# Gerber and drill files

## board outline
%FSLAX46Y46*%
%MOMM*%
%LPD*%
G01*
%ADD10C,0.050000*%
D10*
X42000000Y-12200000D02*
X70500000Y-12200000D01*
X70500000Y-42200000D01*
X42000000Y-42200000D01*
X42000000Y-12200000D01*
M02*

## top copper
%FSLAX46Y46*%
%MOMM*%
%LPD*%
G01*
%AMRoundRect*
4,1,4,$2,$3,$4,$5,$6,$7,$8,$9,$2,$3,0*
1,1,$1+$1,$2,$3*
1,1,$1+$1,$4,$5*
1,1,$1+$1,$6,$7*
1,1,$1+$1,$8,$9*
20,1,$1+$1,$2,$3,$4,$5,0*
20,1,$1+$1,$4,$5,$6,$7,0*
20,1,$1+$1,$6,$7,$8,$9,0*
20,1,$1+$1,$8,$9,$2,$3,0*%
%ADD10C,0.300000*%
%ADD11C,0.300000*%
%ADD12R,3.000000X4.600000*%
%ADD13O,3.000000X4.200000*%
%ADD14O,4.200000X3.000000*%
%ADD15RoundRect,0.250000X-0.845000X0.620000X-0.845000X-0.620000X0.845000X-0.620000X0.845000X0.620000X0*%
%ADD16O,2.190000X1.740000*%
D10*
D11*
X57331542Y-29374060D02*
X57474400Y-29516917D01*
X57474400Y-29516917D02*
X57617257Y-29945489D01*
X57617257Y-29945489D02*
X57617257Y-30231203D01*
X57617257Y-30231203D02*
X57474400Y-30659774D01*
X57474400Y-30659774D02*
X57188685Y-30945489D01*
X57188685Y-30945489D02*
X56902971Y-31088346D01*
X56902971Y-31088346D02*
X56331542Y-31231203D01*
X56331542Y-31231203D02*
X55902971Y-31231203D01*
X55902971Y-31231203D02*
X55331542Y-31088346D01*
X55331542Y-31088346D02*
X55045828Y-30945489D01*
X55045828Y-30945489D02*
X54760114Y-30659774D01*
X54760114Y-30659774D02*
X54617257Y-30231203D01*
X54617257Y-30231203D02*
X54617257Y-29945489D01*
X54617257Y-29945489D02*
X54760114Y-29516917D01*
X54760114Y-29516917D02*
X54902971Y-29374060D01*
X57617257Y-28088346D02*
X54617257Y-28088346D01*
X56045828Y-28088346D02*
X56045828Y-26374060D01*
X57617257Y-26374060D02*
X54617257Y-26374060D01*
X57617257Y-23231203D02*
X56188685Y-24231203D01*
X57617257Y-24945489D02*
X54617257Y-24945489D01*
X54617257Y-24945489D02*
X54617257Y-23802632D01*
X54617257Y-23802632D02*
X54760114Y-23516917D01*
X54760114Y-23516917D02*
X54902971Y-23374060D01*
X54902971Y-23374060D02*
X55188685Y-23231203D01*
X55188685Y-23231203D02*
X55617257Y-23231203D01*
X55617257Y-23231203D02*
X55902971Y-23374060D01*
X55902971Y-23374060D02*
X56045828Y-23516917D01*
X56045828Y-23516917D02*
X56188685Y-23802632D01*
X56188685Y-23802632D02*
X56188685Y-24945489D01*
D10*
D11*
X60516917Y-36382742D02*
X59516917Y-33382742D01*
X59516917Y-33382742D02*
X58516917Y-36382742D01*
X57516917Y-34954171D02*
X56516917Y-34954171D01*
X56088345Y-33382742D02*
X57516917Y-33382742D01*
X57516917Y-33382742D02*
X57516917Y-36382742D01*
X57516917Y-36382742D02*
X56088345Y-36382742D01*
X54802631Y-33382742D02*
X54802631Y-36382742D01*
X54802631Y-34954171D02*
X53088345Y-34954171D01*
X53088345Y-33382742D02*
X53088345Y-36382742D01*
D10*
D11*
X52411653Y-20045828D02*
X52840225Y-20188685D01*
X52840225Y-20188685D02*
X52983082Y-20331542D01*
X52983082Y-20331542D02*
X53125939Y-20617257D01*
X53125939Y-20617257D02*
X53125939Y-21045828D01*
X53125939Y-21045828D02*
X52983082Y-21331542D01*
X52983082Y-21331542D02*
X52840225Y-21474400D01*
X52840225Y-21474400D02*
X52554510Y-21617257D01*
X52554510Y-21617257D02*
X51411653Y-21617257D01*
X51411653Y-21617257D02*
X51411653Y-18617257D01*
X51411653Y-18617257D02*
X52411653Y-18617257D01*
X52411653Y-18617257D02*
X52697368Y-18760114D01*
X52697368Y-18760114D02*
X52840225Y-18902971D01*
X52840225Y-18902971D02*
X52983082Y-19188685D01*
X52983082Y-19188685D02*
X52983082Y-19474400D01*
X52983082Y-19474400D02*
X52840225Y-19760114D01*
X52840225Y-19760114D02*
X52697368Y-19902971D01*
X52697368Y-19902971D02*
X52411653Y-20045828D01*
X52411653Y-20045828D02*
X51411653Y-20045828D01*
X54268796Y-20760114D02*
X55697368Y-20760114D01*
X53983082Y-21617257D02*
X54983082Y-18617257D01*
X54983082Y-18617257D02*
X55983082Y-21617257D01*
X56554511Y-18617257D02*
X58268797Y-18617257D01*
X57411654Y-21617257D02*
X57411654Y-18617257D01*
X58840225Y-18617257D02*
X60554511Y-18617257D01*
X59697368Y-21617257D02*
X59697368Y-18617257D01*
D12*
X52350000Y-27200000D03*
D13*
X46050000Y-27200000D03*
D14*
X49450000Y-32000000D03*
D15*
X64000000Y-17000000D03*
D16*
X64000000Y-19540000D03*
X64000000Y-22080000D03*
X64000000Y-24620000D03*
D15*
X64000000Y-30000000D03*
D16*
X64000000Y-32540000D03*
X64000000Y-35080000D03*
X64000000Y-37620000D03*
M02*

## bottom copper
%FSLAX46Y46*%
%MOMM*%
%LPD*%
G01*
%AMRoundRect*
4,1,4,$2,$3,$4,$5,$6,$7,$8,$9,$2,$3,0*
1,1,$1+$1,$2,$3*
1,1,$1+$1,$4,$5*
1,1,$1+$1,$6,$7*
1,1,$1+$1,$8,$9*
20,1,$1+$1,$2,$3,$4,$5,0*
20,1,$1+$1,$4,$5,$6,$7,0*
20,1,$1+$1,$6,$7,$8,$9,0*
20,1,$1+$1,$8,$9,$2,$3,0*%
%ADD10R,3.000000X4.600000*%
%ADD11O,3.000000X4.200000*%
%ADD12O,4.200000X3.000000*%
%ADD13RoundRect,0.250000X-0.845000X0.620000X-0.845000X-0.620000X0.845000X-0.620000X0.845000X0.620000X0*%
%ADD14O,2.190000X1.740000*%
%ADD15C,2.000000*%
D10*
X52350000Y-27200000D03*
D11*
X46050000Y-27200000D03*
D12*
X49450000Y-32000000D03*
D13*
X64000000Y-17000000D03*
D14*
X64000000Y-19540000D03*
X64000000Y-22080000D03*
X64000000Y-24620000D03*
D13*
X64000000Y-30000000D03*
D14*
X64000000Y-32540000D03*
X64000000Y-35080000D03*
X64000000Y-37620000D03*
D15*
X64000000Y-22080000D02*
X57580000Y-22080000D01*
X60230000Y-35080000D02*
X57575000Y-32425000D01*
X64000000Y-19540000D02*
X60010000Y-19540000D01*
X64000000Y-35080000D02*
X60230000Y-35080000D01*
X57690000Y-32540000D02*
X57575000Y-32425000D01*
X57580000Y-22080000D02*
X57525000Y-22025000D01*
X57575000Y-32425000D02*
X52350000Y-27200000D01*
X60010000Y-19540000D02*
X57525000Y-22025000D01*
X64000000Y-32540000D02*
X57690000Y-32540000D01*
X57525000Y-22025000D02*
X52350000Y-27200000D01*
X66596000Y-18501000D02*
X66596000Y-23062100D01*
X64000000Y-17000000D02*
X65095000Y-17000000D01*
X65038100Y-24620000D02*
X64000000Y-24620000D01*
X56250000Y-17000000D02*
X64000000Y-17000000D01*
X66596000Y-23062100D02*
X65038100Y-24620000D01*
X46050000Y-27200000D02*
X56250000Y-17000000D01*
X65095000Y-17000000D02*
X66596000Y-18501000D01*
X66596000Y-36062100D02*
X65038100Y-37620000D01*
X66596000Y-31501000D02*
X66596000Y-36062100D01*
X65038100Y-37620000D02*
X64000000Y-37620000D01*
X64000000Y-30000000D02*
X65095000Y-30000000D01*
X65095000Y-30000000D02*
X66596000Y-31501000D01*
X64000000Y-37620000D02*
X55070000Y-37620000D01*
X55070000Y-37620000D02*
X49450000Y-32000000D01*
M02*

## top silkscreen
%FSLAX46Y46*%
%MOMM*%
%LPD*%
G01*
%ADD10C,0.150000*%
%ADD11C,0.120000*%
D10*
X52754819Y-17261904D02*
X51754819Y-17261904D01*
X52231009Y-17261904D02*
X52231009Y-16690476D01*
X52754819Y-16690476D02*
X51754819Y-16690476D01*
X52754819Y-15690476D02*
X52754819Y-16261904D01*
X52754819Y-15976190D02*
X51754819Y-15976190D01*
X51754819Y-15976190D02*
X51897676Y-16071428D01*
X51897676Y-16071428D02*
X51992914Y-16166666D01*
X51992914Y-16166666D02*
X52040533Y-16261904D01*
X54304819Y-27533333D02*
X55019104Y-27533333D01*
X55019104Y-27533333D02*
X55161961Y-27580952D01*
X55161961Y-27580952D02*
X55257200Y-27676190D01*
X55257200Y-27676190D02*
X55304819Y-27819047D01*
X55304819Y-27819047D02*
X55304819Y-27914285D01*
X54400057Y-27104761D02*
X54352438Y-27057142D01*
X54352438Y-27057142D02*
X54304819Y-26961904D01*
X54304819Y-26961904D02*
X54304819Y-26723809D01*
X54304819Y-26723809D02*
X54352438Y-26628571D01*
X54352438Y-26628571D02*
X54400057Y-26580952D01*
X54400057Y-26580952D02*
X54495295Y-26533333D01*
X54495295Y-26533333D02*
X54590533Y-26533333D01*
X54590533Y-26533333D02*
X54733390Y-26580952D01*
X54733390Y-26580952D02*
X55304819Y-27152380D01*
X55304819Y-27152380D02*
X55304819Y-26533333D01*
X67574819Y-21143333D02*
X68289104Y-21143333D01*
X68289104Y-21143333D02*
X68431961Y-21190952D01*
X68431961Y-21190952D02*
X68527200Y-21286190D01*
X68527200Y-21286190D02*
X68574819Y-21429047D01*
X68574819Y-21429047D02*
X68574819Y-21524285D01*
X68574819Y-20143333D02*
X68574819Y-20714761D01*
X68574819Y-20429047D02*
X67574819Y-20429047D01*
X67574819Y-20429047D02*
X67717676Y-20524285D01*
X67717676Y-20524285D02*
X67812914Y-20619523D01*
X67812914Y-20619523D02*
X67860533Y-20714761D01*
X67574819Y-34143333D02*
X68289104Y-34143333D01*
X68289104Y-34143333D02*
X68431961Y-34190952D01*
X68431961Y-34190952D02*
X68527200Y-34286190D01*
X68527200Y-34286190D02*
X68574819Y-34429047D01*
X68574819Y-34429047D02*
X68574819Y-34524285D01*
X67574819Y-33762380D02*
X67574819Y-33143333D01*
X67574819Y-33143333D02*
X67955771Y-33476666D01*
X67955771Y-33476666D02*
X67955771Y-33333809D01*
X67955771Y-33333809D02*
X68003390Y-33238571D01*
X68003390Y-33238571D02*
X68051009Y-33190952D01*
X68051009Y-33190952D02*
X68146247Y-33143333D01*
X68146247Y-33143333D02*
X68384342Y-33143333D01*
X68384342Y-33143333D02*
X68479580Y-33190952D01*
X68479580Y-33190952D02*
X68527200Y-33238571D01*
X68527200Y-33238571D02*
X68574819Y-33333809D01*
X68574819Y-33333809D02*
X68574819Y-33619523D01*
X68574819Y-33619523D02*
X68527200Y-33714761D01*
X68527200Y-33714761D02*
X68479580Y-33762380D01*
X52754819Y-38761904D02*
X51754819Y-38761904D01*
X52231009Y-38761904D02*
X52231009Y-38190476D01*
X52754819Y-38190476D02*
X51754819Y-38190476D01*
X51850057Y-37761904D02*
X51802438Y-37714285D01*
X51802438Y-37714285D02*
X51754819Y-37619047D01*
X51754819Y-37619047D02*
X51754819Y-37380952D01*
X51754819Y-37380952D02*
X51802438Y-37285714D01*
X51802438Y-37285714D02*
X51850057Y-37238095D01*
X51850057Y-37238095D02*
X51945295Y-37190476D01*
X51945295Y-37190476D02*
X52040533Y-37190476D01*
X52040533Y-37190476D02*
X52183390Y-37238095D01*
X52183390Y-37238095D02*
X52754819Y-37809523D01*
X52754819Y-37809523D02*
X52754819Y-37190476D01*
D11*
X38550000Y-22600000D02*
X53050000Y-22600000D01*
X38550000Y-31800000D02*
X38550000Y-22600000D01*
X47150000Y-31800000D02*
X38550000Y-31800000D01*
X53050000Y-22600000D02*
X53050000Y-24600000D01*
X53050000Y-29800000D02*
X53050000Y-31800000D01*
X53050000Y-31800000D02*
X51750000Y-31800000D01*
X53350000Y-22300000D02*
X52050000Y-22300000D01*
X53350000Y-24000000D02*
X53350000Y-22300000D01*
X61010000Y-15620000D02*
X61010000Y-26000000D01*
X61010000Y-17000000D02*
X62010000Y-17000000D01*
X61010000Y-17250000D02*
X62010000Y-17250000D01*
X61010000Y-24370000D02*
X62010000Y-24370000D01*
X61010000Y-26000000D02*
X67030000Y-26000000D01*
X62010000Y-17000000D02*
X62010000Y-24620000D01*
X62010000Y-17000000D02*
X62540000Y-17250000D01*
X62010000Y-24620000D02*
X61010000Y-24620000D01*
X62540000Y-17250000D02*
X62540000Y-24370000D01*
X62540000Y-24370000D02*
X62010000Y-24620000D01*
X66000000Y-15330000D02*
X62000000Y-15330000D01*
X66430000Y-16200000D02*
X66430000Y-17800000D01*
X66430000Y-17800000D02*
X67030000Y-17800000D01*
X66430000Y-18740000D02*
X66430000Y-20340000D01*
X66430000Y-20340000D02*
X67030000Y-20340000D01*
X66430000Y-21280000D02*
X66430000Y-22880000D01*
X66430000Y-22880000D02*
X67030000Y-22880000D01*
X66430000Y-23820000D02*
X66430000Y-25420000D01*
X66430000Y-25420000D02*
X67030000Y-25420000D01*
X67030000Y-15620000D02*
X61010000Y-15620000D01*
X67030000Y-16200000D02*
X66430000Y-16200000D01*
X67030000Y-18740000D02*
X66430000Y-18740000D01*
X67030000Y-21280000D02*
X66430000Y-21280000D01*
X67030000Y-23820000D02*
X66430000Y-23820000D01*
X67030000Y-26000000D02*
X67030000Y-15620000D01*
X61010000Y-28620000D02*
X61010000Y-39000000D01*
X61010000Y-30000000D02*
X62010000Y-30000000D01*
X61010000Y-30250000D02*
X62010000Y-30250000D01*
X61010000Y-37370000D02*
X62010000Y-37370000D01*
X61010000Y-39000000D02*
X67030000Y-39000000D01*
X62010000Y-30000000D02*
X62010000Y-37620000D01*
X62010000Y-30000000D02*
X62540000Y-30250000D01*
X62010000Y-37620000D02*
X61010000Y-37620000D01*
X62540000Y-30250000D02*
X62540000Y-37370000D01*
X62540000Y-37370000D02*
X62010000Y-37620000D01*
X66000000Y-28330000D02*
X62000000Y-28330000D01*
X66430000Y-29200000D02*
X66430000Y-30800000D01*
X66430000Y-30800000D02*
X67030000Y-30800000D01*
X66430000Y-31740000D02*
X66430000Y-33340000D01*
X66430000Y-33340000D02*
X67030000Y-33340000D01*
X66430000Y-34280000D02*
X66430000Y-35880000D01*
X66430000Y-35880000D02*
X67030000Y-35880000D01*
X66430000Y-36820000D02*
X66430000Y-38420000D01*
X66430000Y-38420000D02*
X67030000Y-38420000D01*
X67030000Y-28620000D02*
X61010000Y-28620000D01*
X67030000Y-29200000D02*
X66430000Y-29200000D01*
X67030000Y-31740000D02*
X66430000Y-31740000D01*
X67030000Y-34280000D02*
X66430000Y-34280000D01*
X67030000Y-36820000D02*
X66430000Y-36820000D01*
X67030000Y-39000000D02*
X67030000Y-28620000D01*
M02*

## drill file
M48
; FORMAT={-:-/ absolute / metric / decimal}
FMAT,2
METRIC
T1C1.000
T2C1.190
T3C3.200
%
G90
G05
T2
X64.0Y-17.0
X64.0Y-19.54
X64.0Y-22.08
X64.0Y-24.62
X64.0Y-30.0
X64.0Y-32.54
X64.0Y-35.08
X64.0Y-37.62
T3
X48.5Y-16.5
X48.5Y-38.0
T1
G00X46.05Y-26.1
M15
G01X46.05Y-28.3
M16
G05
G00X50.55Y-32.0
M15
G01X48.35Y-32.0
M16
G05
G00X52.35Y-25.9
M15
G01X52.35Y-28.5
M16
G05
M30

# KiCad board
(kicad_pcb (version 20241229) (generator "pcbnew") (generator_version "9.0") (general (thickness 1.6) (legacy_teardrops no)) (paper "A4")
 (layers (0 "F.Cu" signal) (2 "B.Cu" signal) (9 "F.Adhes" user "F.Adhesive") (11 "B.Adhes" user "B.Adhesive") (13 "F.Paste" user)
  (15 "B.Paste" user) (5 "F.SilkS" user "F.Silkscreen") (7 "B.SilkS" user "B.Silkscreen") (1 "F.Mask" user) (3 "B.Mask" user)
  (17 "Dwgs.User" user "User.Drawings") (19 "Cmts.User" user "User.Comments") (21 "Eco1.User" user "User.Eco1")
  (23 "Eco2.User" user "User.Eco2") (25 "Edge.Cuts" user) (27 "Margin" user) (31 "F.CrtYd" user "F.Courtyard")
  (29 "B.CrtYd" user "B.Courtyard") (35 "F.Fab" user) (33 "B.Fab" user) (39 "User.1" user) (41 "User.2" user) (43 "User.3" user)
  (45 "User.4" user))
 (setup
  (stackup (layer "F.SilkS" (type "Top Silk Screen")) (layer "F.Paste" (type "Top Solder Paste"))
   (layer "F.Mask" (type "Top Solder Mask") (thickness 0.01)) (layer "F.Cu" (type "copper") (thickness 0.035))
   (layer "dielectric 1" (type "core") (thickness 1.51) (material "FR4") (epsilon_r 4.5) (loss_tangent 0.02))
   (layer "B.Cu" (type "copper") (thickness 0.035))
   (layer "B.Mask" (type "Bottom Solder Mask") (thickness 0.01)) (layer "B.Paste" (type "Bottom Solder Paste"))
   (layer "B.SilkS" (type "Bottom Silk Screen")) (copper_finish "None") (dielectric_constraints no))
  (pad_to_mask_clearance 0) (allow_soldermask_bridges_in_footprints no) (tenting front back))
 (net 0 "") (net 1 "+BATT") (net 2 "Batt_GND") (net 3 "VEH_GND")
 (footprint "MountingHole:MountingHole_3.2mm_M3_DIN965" (layer "F.Cu") (at 48.5 16.5 -90)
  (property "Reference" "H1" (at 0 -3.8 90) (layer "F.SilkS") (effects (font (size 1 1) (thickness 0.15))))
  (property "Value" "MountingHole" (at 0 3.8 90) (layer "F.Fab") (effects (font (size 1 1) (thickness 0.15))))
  (pad "" np_thru_hole circle (at 0 0 270) (size 3.2 3.2) (drill 3.2) (layers "*.Cu" "*.Mask")))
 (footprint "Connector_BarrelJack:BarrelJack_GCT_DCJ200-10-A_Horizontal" (layer "F.Cu") (at 52.35 27.2 -90)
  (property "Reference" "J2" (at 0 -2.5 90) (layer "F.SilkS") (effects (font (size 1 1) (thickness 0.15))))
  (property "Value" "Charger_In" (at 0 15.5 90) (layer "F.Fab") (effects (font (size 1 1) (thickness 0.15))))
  (fp_line (start -4.6 13.8) (end -4.6 -0.7) (stroke (width 0.12) (type solid)) (layer "F.SilkS"))
  (fp_line (start 4.6 13.8) (end -4.6 13.8) (stroke (width 0.12) (type solid)) (layer "F.SilkS"))
  (fp_line (start 4.6 5.2) (end 4.6 13.8) (stroke (width 0.12) (type solid)) (layer "F.SilkS"))
  (fp_line (start -4.6 -0.7) (end -2.6 -0.7) (stroke (width 0.12) (type solid)) (layer "F.SilkS"))
  (fp_line (start 2.6 -0.7) (end 4.6 -0.7) (stroke (width 0.12) (type solid)) (layer "F.SilkS"))
  (fp_line (start 4.6 -0.7) (end 4.6 0.6) (stroke (width 0.12) (type solid)) (layer "F.SilkS"))
  (fp_line (start -4.9 -1) (end -4.9 0.3) (stroke (width 0.12) (type solid)) (layer "F.SilkS"))
  (fp_line (start -3.2 -1) (end -4.9 -1) (stroke (width 0.12) (type solid)) (layer "F.SilkS"))
  (pad "1" thru_hole rect (at 0 0 270) (size 4.6 3) (drill oval 3.6 1) (layers "*.Cu" "*.Mask") (remove_unused_layers no) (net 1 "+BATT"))
  (pad "2" thru_hole oval (at 0 6.3 270) (size 4.2 3) (drill oval 3.2 1) (layers "*.Cu" "*.Mask") (remove_unused_layers no)
   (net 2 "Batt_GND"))
  (pad "3" thru_hole oval (at 4.8 2.9 270) (size 3 4.2) (drill oval 1 3.2) (layers "*.Cu" "*.Mask") (remove_unused_layers no)
   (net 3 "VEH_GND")))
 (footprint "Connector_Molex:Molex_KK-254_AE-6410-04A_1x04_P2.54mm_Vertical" (layer "F.Cu") (at 64 17 -90)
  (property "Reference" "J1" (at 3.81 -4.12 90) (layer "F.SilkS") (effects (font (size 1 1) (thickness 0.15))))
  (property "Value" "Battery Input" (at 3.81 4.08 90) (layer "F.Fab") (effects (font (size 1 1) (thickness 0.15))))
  (fp_line (start -1.38 2.99) (end 9 2.99) (stroke (width 0.12) (type solid)) (layer "F.SilkS"))
  (fp_line (start 0 2.99) (end 0 1.99) (stroke (width 0.12) (type solid)) (layer "F.SilkS"))
  (fp_line (start 0.25 2.99) (end 0.25 1.99) (stroke (width 0.12) (type solid)) (layer "F.SilkS"))
  (fp_line (start 7.37 2.99) (end 7.37 1.99) (stroke (width 0.12) (type solid)) (layer "F.SilkS"))
  (fp_line (start 9 2.99) (end 9 -3.03) (stroke (width 0.12) (type solid)) (layer "F.SilkS"))
  (fp_line (start 0 1.99) (end 7.62 1.99) (stroke (width 0.12) (type solid)) (layer "F.SilkS"))
  (fp_line (start 0 1.99) (end 0.25 1.46) (stroke (width 0.12) (type solid)) (layer "F.SilkS"))
  (fp_line (start 7.62 1.99) (end 7.62 2.99) (stroke (width 0.12) (type solid)) (layer "F.SilkS"))
  (fp_line (start 0.25 1.46) (end 7.37 1.46) (stroke (width 0.12) (type solid)) (layer "F.SilkS"))
  (fp_line (start 7.37 1.46) (end 7.62 1.99) (stroke (width 0.12) (type solid)) (layer "F.SilkS"))
  (fp_line (start -1.67 -2) (end -1.67 2) (stroke (width 0.12) (type solid)) (layer "F.SilkS"))
  (fp_line (start -0.8 -2.43) (end 0.8 -2.43) (stroke (width 0.12) (type solid)) (layer "F.SilkS"))
  (fp_line (start 0.8 -2.43) (end 0.8 -3.03) (stroke (width 0.12) (type solid)) (layer "F.SilkS"))
  (fp_line (start 1.74 -2.43) (end 3.34 -2.43) (stroke (width 0.12) (type solid)) (layer "F.SilkS"))
  (fp_line (start 3.34 -2.43) (end 3.34 -3.03) (stroke (width 0.12) (type solid)) (layer "F.SilkS"))
  (fp_line (start 4.28 -2.43) (end 5.88 -2.43) (stroke (width 0.12) (type solid)) (layer "F.SilkS"))
  (fp_line (start 5.88 -2.43) (end 5.88 -3.03) (stroke (width 0.12) (type solid)) (layer "F.SilkS"))
  (fp_line (start 6.82 -2.43) (end 8.42 -2.43) (stroke (width 0.12) (type solid)) (layer "F.SilkS"))
  (fp_line (start 8.42 -2.43) (end 8.42 -3.03) (stroke (width 0.12) (type solid)) (layer "F.SilkS"))
  (fp_line (start -1.38 -3.03) (end -1.38 2.99) (stroke (width 0.12) (type solid)) (layer "F.SilkS"))
  (fp_line (start -0.8 -3.03) (end -0.8 -2.43) (stroke (width 0.12) (type solid)) (layer "F.SilkS"))
  (fp_line (start 1.74 -3.03) (end 1.74 -2.43) (stroke (width 0.12) (type solid)) (layer "F.SilkS"))
  (fp_line (start 4.28 -3.03) (end 4.28 -2.43) (stroke (width 0.12) (type solid)) (layer "F.SilkS"))
  (fp_line (start 6.82 -3.03) (end 6.82 -2.43) (stroke (width 0.12) (type solid)) (layer "F.SilkS"))
  (fp_line (start 9 -3.03) (end -1.38 -3.03) (stroke (width 0.12) (type solid)) (layer "F.SilkS"))
  (pad "1" thru_hole roundrect (at 0 0 270) (size 1.74 2.19) (drill 1.19) (layers "*.Cu" "*.Mask") (remove_unused_layers no)
   (roundrect_rratio 0.143678) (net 2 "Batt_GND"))
  (pad "2" thru_hole oval (at 2.54 0 270) (size 1.74 2.19) (drill 1.19) (layers "*.Cu" "*.Mask") (remove_unused_layers no) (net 1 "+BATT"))
  (pad "3" thru_hole oval (at 5.08 0 270) (size 1.74 2.19) (drill 1.19) (layers "*.Cu" "*.Mask") (remove_unused_layers no) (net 1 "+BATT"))
  (pad "4" thru_hole oval (at 7.62 0 270) (size 1.74 2.19) (drill 1.19) (layers "*.Cu" "*.Mask") (remove_unused_layers no)
   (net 2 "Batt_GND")))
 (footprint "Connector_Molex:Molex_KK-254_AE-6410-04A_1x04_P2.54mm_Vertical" (layer "F.Cu") (at 64 30 -90)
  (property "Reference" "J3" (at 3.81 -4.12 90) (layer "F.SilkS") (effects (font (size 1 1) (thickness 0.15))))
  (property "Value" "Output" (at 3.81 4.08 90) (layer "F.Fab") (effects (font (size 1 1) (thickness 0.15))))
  (fp_line (start -1.38 2.99) (end 9 2.99) (stroke (width 0.12) (type solid)) (layer "F.SilkS"))
  (fp_line (start 0 2.99) (end 0 1.99) (stroke (width 0.12) (type solid)) (layer "F.SilkS"))
  (fp_line (start 0.25 2.99) (end 0.25 1.99) (stroke (width 0.12) (type solid)) (layer "F.SilkS"))
  (fp_line (start 7.37 2.99) (end 7.37 1.99) (stroke (width 0.12) (type solid)) (layer "F.SilkS"))
  (fp_line (start 9 2.99) (end 9 -3.03) (stroke (width 0.12) (type solid)) (layer "F.SilkS"))
  (fp_line (start 0 1.99) (end 7.62 1.99) (stroke (width 0.12) (type solid)) (layer "F.SilkS"))
  (fp_line (start 0 1.99) (end 0.25 1.46) (stroke (width 0.12) (type solid)) (layer "F.SilkS"))
  (fp_line (start 7.62 1.99) (end 7.62 2.99) (stroke (width 0.12) (type solid)) (layer "F.SilkS"))
  (fp_line (start 0.25 1.46) (end 7.37 1.46) (stroke (width 0.12) (type solid)) (layer "F.SilkS"))
  (fp_line (start 7.37 1.46) (end 7.62 1.99) (stroke (width 0.12) (type solid)) (layer "F.SilkS"))
  (fp_line (start -1.67 -2) (end -1.67 2) (stroke (width 0.12) (type solid)) (layer "F.SilkS"))
  (fp_line (start -0.8 -2.43) (end 0.8 -2.43) (stroke (width 0.12) (type solid)) (layer "F.SilkS"))
  (fp_line (start 0.8 -2.43) (end 0.8 -3.03) (stroke (width 0.12) (type solid)) (layer "F.SilkS"))
  (fp_line (start 1.74 -2.43) (end 3.34 -2.43) (stroke (width 0.12) (type solid)) (layer "F.SilkS"))
  (fp_line (start 3.34 -2.43) (end 3.34 -3.03) (stroke (width 0.12) (type solid)) (layer "F.SilkS"))
  (fp_line (start 4.28 -2.43) (end 5.88 -2.43) (stroke (width 0.12) (type solid)) (layer "F.SilkS"))
  (fp_line (start 5.88 -2.43) (end 5.88 -3.03) (stroke (width 0.12) (type solid)) (layer "F.SilkS"))
  (fp_line (start 6.82 -2.43) (end 8.42 -2.43) (stroke (width 0.12) (type solid)) (layer "F.SilkS"))
  (fp_line (start 8.42 -2.43) (end 8.42 -3.03) (stroke (width 0.12) (type solid)) (layer "F.SilkS"))
  (fp_line (start -1.38 -3.03) (end -1.38 2.99) (stroke (width 0.12) (type solid)) (layer "F.SilkS"))
  (fp_line (start -0.8 -3.03) (end -0.8 -2.43) (stroke (width 0.12) (type solid)) (layer "F.SilkS"))
  (fp_line (start 1.74 -3.03) (end 1.74 -2.43) (stroke (width 0.12) (type solid)) (layer "F.SilkS"))
  (fp_line (start 4.28 -3.03) (end 4.28 -2.43) (stroke (width 0.12) (type solid)) (layer "F.SilkS"))
  (fp_line (start 6.82 -3.03) (end 6.82 -2.43) (stroke (width 0.12) (type solid)) (layer "F.SilkS"))
  (fp_line (start 9 -3.03) (end -1.38 -3.03) (stroke (width 0.12) (type solid)) (layer "F.SilkS"))
  (pad "1" thru_hole roundrect (at 0 0 270) (size 1.74 2.19) (drill 1.19) (layers "*.Cu" "*.Mask") (remove_unused_layers no)
   (roundrect_rratio 0.143678) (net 3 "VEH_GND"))
  (pad "2" thru_hole oval (at 2.54 0 270) (size 1.74 2.19) (drill 1.19) (layers "*.Cu" "*.Mask") (remove_unused_layers no) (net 1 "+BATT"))
  (pad "3" thru_hole oval (at 5.08 0 270) (size 1.74 2.19) (drill 1.19) (layers "*.Cu" "*.Mask") (remove_unused_layers no) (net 1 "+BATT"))
  (pad "4" thru_hole oval (at 7.62 0 270) (size 1.74 2.19) (drill 1.19) (layers "*.Cu" "*.Mask") (remove_unused_layers no) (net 3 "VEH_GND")))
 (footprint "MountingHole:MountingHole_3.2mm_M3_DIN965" (layer "F.Cu") (at 48.5 38 -90)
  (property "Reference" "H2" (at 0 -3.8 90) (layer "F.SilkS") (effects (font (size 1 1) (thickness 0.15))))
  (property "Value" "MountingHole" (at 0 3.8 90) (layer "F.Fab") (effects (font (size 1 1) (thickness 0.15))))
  (pad "" np_thru_hole circle (at 0 0 270) (size 3.2 3.2) (drill 3.2) (layers "*.Cu" "*.Mask")))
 (gr_rect (start 42 12.2) (end 70.5 42.2) (stroke (width 0.05) (type solid)) (fill no) (layer "Edge.Cuts"))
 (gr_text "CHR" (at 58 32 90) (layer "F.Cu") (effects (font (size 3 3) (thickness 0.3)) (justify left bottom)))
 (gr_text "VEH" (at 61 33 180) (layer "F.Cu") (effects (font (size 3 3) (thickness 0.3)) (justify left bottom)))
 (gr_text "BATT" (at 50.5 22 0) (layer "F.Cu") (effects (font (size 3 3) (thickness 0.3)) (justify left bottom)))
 (segment (start 64 22.08) (end 57.58 22.08) (width 2) (layer "B.Cu") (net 1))
 (segment (start 60.23 35.08) (end 57.575 32.425) (width 2) (layer "B.Cu") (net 1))
 (segment (start 64 19.54) (end 60.01 19.54) (width 2) (layer "B.Cu") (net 1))
 (segment (start 64 35.08) (end 60.23 35.08) (width 2) (layer "B.Cu") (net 1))
 (segment (start 57.69 32.54) (end 57.575 32.425) (width 2) (layer "B.Cu") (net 1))
 (segment (start 57.58 22.08) (end 57.525 22.025) (width 2) (layer "B.Cu") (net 1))
 (segment (start 57.575 32.425) (end 52.35 27.2) (width 2) (layer "B.Cu") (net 1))
 (segment (start 60.01 19.54) (end 57.525 22.025) (width 2) (layer "B.Cu") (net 1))
 (segment (start 64 32.54) (end 57.69 32.54) (width 2) (layer "B.Cu") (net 1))
 (segment (start 57.525 22.025) (end 52.35 27.2) (width 2) (layer "B.Cu") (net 1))
 (segment (start 66.596 18.501) (end 66.596 23.0621) (width 2) (layer "B.Cu") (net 2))
 (segment (start 64 17) (end 65.095 17) (width 2) (layer "B.Cu") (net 2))
 (segment (start 65.0381 24.62) (end 64 24.62) (width 2) (layer "B.Cu") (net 2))
 (segment (start 56.25 17) (end 64 17) (width 2) (layer "B.Cu") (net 2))
 (segment (start 66.596 23.0621) (end 65.0381 24.62) (width 2) (layer "B.Cu") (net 2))
 (segment (start 46.05 27.2) (end 56.25 17) (width 2) (layer "B.Cu") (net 2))
 (segment (start 65.095 17) (end 66.596 18.501) (width 2) (layer "B.Cu") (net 2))
 (segment (start 66.596 36.0621) (end 65.0381 37.62) (width 2) (layer "B.Cu") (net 3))
 (segment (start 66.596 31.501) (end 66.596 36.0621) (width 2) (layer "B.Cu") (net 3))
 (segment (start 65.0381 37.62) (end 64 37.62) (width 2) (layer "B.Cu") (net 3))
 (segment (start 64 30) (end 65.095 30) (width 2) (layer "B.Cu") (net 3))
 (segment (start 65.095 30) (end 66.596 31.501) (width 2) (layer "B.Cu") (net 3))
 (segment (start 64 37.62) (end 55.07 37.62) (width 2) (layer "B.Cu") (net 3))
 (segment (start 55.07 37.62) (end 49.45 32) (width 2) (layer "B.Cu") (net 3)))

